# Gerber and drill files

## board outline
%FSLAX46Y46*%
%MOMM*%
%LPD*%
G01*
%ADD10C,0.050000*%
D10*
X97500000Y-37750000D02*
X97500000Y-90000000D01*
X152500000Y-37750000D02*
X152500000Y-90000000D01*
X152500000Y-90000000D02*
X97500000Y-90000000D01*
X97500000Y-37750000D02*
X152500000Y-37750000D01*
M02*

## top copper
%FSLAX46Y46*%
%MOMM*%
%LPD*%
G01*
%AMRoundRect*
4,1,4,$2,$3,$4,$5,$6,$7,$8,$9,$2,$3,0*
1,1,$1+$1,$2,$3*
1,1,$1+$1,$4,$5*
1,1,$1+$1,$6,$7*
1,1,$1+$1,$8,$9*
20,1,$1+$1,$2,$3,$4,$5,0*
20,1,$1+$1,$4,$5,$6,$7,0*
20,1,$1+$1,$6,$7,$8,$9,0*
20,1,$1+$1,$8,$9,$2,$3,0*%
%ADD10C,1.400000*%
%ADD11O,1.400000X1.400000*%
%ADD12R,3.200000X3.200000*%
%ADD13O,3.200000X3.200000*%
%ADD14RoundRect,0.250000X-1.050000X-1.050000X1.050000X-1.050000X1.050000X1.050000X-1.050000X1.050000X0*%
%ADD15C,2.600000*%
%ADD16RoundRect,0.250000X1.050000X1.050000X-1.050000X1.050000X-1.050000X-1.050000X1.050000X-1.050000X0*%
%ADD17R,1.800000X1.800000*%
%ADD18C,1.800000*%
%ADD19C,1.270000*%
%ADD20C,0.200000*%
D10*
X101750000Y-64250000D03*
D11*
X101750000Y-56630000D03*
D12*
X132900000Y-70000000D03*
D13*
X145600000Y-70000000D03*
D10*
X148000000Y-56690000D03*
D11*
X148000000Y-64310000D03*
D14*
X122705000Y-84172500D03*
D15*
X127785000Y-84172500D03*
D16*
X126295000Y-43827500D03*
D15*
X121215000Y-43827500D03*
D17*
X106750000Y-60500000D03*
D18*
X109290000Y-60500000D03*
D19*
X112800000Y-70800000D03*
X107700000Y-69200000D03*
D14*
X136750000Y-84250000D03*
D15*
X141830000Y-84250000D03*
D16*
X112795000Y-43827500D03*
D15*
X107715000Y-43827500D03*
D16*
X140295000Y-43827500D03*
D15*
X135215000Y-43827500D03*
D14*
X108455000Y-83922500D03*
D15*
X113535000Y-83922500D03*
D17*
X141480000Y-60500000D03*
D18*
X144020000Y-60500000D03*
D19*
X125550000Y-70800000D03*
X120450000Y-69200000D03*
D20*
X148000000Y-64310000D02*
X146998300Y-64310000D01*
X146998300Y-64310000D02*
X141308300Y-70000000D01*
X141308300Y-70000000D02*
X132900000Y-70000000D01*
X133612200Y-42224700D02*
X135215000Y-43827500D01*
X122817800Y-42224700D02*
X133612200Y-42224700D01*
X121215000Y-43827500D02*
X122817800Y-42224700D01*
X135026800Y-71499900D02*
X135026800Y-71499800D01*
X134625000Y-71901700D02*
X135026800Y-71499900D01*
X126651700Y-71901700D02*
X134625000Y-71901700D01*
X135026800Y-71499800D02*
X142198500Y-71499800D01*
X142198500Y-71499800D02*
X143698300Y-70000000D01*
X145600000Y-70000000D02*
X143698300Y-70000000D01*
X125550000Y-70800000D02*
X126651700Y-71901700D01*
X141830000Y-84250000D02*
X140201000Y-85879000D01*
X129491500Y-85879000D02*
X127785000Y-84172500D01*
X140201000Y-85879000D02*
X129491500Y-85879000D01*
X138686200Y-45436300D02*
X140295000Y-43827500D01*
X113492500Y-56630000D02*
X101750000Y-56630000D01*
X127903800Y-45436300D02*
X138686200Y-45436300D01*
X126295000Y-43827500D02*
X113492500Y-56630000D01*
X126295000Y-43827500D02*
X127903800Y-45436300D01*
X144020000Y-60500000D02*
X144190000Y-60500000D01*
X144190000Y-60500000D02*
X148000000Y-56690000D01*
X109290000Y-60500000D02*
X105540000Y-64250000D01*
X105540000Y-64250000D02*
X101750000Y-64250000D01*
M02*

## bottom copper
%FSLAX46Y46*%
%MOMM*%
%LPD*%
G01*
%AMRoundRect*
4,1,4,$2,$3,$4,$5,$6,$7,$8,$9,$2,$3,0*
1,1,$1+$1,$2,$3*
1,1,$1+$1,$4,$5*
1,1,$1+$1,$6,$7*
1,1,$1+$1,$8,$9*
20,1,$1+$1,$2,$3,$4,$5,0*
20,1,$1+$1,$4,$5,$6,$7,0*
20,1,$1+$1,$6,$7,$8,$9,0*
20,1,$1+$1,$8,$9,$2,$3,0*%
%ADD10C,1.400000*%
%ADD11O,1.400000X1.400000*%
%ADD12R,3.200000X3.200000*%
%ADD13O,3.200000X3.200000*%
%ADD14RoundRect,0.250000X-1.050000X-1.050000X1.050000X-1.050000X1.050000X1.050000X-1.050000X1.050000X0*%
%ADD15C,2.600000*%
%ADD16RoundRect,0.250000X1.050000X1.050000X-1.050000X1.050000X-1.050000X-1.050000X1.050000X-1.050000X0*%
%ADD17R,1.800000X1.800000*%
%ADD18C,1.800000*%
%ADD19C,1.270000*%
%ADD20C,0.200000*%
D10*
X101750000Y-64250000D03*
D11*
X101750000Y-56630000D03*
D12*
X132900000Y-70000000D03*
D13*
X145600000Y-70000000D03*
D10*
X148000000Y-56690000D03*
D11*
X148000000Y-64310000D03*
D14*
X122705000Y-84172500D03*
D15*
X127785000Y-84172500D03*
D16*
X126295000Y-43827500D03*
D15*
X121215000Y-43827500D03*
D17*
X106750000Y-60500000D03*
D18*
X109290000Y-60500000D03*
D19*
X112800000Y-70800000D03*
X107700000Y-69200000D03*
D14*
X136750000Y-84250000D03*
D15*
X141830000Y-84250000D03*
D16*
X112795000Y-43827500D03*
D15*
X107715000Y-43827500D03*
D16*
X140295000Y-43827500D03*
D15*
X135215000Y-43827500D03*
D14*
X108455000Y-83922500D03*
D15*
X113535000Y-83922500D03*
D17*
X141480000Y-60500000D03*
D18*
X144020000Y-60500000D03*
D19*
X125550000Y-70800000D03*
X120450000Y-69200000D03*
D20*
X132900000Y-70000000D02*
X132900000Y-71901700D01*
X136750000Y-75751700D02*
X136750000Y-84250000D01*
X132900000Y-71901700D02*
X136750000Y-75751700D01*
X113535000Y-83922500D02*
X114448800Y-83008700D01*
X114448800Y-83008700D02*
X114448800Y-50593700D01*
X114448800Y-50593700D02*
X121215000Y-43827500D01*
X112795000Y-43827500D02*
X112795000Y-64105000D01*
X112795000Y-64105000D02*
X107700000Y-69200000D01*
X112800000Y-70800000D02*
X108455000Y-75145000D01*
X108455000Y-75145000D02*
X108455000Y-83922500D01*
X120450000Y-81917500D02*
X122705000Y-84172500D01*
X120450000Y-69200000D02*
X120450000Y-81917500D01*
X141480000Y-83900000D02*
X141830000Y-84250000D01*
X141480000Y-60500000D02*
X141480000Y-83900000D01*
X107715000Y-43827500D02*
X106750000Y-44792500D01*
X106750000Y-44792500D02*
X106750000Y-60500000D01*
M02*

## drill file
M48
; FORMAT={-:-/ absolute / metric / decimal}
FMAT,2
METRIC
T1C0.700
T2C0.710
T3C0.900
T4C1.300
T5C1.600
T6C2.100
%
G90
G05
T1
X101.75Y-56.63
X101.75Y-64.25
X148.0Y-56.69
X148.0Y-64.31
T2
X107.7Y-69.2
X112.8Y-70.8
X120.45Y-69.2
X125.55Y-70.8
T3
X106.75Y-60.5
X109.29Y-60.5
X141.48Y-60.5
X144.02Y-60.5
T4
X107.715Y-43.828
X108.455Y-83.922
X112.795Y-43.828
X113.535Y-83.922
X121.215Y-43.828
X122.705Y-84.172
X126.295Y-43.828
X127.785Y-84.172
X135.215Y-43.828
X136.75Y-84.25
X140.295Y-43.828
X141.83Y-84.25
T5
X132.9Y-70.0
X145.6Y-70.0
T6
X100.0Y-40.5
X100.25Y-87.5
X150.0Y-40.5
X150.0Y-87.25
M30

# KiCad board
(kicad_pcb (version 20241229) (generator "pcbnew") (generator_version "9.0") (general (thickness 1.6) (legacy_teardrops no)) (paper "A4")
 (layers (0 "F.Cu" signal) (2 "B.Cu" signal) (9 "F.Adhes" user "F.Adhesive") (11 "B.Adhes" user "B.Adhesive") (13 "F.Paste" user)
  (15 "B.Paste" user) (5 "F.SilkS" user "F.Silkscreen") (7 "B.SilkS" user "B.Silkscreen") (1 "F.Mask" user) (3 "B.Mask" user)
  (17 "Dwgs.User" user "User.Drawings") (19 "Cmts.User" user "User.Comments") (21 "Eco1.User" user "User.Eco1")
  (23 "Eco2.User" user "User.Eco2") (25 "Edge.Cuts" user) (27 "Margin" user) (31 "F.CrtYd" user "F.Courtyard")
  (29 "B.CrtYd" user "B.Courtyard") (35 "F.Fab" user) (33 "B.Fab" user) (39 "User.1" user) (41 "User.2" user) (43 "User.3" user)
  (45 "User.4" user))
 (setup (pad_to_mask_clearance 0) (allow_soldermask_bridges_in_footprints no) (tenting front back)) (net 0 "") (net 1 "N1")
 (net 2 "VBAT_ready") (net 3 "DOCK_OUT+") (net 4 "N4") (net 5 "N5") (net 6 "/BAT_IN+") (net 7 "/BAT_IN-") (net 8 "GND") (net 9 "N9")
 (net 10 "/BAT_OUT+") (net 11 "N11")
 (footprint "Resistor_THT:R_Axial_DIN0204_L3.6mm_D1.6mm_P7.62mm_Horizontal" (layer "F.Cu") (at 101.75 64.25 90)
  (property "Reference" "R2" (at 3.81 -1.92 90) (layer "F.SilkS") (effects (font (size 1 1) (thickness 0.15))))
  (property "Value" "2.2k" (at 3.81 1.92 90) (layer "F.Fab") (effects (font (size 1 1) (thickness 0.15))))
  (pad "1" thru_hole circle (at 0 0 90) (size 1.4 1.4) (drill 0.7) (layers "*.Cu" "*.Mask") (remove_unused_layers no) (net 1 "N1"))
  (pad "2" thru_hole oval (at 7.62 0 90) (size 1.4 1.4) (drill 0.7) (layers "*.Cu" "*.Mask") (remove_unused_layers no) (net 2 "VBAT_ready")))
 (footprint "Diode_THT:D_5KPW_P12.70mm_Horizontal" (layer "F.Cu") (at 132.9 70)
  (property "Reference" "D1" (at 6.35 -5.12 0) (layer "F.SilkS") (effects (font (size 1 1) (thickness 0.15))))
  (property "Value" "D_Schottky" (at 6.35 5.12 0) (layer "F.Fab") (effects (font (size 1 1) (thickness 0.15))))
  (pad "1" thru_hole rect (at 0 0) (size 3.2 3.2) (drill 1.6) (layers "*.Cu" "*.Mask") (remove_unused_layers no) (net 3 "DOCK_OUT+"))
  (pad "2" thru_hole oval (at 12.7 0) (size 3.2 3.2) (drill 1.6) (layers "*.Cu" "*.Mask") (remove_unused_layers no) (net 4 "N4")))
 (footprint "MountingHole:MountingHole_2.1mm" (layer "F.Cu") (at 100.25 87.5)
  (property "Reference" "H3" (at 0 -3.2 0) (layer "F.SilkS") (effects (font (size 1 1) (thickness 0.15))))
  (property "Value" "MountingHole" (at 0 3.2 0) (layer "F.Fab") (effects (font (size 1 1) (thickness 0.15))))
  (pad "" np_thru_hole circle (at 0 0) (size 2.1 2.1) (drill 2.1) (layers "*.Cu" "*.Mask")))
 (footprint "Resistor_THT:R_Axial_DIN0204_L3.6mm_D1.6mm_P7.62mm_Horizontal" (layer "F.Cu") (at 148 56.69 -90)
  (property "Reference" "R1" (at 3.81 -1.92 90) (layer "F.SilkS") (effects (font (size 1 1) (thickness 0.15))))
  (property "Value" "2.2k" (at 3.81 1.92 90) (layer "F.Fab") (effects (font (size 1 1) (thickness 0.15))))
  (pad "1" thru_hole circle (at 0 0 270) (size 1.4 1.4) (drill 0.7) (layers "*.Cu" "*.Mask") (remove_unused_layers no) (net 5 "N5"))
  (pad "2" thru_hole oval (at 7.62 0 270) (size 1.4 1.4) (drill 0.7) (layers "*.Cu" "*.Mask") (remove_unused_layers no) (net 3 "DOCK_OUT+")))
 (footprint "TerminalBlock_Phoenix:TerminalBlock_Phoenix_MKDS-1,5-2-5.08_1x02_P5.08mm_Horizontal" (layer "F.Cu") (at 122.705 84.1725)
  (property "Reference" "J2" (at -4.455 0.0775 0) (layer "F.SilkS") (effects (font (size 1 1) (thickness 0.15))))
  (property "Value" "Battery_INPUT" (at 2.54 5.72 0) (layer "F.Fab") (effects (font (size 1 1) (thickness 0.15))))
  (pad "1" thru_hole roundrect (at 0 0) (size 2.6 2.6) (drill 1.3) (layers "*.Cu" "*.Mask") (remove_unused_layers no)
   (roundrect_rratio 0.096154) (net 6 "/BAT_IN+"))
  (pad "2" thru_hole circle (at 5.08 0) (size 2.6 2.6) (drill 1.3) (layers "*.Cu" "*.Mask") (remove_unused_layers no) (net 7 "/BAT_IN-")))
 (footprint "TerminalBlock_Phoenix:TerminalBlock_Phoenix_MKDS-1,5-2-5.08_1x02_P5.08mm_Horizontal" (layer "F.Cu") (at 126.295 43.8275 180)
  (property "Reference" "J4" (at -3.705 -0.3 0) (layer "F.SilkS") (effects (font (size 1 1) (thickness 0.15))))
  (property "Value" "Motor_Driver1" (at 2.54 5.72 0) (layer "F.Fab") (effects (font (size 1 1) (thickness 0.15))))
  (pad "1" thru_hole roundrect (at 0 0 180) (size 2.6 2.6) (drill 1.3) (layers "*.Cu" "*.Mask") (remove_unused_layers no)
   (roundrect_rratio 0.096154) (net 2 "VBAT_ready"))
  (pad "2" thru_hole circle (at 5.08 0 180) (size 2.6 2.6) (drill 1.3) (layers "*.Cu" "*.Mask") (remove_unused_layers no) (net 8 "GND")))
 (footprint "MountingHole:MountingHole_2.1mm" (layer "F.Cu") (at 150 40.5)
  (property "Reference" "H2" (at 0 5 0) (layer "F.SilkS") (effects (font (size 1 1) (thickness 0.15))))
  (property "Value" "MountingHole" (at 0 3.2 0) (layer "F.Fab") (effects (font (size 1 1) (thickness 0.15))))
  (pad "" np_thru_hole circle (at 0 0) (size 2.1 2.1) (drill 2.1) (layers "*.Cu" "*.Mask")))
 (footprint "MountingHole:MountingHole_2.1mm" (layer "F.Cu") (at 100 40.5)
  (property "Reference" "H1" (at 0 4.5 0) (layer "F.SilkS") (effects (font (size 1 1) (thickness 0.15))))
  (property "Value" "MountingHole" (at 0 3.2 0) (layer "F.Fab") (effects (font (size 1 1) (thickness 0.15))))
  (pad "" np_thru_hole circle (at 0 0) (size 2.1 2.1) (drill 2.1) (layers "*.Cu" "*.Mask")))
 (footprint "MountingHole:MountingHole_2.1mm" (layer "F.Cu") (at 150 87.25)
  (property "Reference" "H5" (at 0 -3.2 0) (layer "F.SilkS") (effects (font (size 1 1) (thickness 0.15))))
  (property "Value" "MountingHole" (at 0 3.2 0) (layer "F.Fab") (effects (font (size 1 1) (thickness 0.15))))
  (pad "" np_thru_hole circle (at 0 0) (size 2.1 2.1) (drill 2.1) (layers "*.Cu" "*.Mask")))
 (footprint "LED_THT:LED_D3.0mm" (layer "F.Cu") (at 106.75 60.5)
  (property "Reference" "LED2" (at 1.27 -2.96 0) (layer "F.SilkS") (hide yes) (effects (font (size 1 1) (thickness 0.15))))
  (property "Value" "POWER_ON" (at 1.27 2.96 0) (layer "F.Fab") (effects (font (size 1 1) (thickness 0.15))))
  (pad "1" thru_hole rect (at 0 0) (size 1.8 1.8) (drill 0.9) (layers "*.Cu" "*.Mask") (remove_unused_layers no) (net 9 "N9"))
  (pad "2" thru_hole circle (at 2.54 0) (size 1.8 1.8) (drill 0.9) (layers "*.Cu" "*.Mask") (remove_unused_layers no) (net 1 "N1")))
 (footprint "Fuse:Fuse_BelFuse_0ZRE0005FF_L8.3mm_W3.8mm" (layer "F.Cu") (at 112.8 70.8 180)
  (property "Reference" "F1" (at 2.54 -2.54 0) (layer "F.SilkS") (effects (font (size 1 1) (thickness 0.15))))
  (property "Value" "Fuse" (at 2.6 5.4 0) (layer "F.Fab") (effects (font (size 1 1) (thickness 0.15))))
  (pad "1" thru_hole circle (at 0 0 180) (size 1.27 1.27) (drill 0.71) (layers "*.Cu" "*.Mask") (remove_unused_layers no)
   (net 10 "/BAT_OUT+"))
  (pad "2" thru_hole circle (at 5.1 1.6 180) (size 1.27 1.27) (drill 0.71) (layers "*.Cu" "*.Mask") (remove_unused_layers no) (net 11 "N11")))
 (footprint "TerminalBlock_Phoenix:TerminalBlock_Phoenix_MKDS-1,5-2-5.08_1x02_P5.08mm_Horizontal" (layer "F.Cu") (at 136.75 84.25)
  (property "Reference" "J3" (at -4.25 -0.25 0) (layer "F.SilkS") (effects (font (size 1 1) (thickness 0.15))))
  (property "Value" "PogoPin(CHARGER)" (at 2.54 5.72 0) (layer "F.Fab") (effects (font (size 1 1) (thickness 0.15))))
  (pad "1" thru_hole roundrect (at 0 0) (size 2.6 2.6) (drill 1.3) (layers "*.Cu" "*.Mask") (remove_unused_layers no)
   (roundrect_rratio 0.096154) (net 3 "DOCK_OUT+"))
  (pad "2" thru_hole circle (at 5.08 0) (size 2.6 2.6) (drill 1.3) (layers "*.Cu" "*.Mask") (remove_unused_layers no) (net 7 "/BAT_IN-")))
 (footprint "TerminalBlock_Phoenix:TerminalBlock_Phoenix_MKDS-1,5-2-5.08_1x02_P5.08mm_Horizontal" (layer "F.Cu") (at 112.795 43.8275 180)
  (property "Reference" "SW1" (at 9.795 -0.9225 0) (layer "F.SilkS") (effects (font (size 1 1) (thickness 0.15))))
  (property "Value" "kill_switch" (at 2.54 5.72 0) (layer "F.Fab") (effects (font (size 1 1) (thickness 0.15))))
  (pad "1" thru_hole roundrect (at 0 0 180) (size 2.6 2.6) (drill 1.3) (layers "*.Cu" "*.Mask") (remove_unused_layers no)
   (roundrect_rratio 0.096154) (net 11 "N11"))
  (pad "2" thru_hole circle (at 5.08 0 180) (size 2.6 2.6) (drill 1.3) (layers "*.Cu" "*.Mask") (remove_unused_layers no) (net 9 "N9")))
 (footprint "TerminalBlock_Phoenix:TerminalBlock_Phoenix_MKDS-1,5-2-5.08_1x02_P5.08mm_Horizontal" (layer "F.Cu") (at 140.295 43.8275 180)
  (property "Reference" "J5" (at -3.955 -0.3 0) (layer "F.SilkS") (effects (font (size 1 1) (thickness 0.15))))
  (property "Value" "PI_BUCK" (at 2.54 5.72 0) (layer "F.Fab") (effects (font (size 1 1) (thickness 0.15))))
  (pad "1" thru_hole roundrect (at 0 0 180) (size 2.6 2.6) (drill 1.3) (layers "*.Cu" "*.Mask") (remove_unused_layers no)
   (roundrect_rratio 0.096154) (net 2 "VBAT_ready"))
  (pad "2" thru_hole circle (at 5.08 0 180) (size 2.6 2.6) (drill 1.3) (layers "*.Cu" "*.Mask") (remove_unused_layers no) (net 8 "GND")))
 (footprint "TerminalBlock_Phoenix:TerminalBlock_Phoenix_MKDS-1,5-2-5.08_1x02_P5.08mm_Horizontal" (layer "F.Cu") (at 108.455 83.9225)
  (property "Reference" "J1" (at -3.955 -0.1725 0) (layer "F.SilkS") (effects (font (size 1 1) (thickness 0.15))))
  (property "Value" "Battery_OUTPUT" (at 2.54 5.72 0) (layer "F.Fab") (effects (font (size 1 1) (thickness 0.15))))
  (pad "1" thru_hole roundrect (at 0 0) (size 2.6 2.6) (drill 1.3) (layers "*.Cu" "*.Mask") (remove_unused_layers no)
   (roundrect_rratio 0.096154) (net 10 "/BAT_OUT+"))
  (pad "2" thru_hole circle (at 5.08 0) (size 2.6 2.6) (drill 1.3) (layers "*.Cu" "*.Mask") (remove_unused_layers no) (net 8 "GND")))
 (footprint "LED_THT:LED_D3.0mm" (layer "F.Cu") (at 141.48 60.5)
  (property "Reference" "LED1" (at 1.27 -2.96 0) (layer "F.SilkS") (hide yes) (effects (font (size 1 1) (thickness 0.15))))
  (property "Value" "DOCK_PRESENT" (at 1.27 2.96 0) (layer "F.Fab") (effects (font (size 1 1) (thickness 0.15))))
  (pad "1" thru_hole rect (at 0 0) (size 1.8 1.8) (drill 0.9) (layers "*.Cu" "*.Mask") (remove_unused_layers no) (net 7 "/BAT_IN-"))
  (pad "2" thru_hole circle (at 2.54 0) (size 1.8 1.8) (drill 0.9) (layers "*.Cu" "*.Mask") (remove_unused_layers no) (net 5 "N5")))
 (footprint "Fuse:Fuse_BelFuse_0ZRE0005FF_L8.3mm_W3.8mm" (layer "F.Cu") (at 125.55 70.8 180)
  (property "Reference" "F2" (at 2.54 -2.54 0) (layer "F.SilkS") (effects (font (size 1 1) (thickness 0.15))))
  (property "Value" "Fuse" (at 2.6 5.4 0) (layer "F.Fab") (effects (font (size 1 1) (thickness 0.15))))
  (pad "1" thru_hole circle (at 0 0 180) (size 1.27 1.27) (drill 0.71) (layers "*.Cu" "*.Mask") (remove_unused_layers no) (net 4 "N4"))
  (pad "2" thru_hole circle (at 5.1 1.6 180) (size 1.27 1.27) (drill 0.71) (layers "*.Cu" "*.Mask") (remove_unused_layers no)
   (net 6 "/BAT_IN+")))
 (gr_line (start 97.5 37.75) (end 97.5 90) (stroke (width 0.05) (type default)) (layer "Edge.Cuts"))
 (gr_line (start 152.5 37.75) (end 152.5 90) (stroke (width 0.05) (type default)) (layer "Edge.Cuts"))
 (gr_line (start 152.5 90) (end 97.5 90) (stroke (width 0.05) (type default)) (layer "Edge.Cuts"))
 (gr_line (start 97.5 37.75) (end 152.5 37.75) (stroke (width 0.05) (type default)) (layer "Edge.Cuts"))
 (segment (start 148 64.31) (end 146.9983 64.31) (width 0.2) (layer "F.Cu") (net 3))
 (segment (start 146.9983 64.31) (end 141.3083 70) (width 0.2) (layer "F.Cu") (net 3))
 (segment (start 141.3083 70) (end 132.9 70) (width 0.2) (layer "F.Cu") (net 3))
 (segment (start 132.9 70) (end 132.9 71.9017) (width 0.2) (layer "B.Cu") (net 3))
 (segment (start 136.75 75.7517) (end 136.75 84.25) (width 0.2) (layer "B.Cu") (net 3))
 (segment (start 132.9 71.9017) (end 136.75 75.7517) (width 0.2) (layer "B.Cu") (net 3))
 (segment (start 133.6122 42.2247) (end 135.215 43.8275) (width 0.2) (layer "F.Cu") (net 8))
 (segment (start 122.8178 42.2247) (end 133.6122 42.2247) (width 0.2) (layer "F.Cu") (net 8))
 (segment (start 121.215 43.8275) (end 122.8178 42.2247) (width 0.2) (layer "F.Cu") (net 8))
 (segment (start 113.535 83.9225) (end 114.4488 83.0087) (width 0.2) (layer "B.Cu") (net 8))
 (segment (start 114.4488 83.0087) (end 114.4488 50.5937) (width 0.2) (layer "B.Cu") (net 8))
 (segment (start 114.4488 50.5937) (end 121.215 43.8275) (width 0.2) (layer "B.Cu") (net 8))
 (segment (start 135.0268 71.4999) (end 135.0268 71.4998) (width 0.2) (layer "F.Cu") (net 4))
 (segment (start 134.625 71.9017) (end 135.0268 71.4999) (width 0.2) (layer "F.Cu") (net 4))
 (segment (start 126.6517 71.9017) (end 134.625 71.9017) (width 0.2) (layer "F.Cu") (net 4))
 (segment (start 135.0268 71.4998) (end 142.1985 71.4998) (width 0.2) (layer "F.Cu") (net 4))
 (segment (start 142.1985 71.4998) (end 143.6983 70) (width 0.2) (layer "F.Cu") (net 4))
 (segment (start 145.6 70) (end 143.6983 70) (width 0.2) (layer "F.Cu") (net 4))
 (segment (start 125.55 70.8) (end 126.6517 71.9017) (width 0.2) (layer "F.Cu") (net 4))
 (segment (start 112.795 43.8275) (end 112.795 64.105) (width 0.2) (layer "B.Cu") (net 11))
 (segment (start 112.795 64.105) (end 107.7 69.2) (width 0.2) (layer "B.Cu") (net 11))
 (segment (start 112.8 70.8) (end 108.455 75.145) (width 0.2) (layer "B.Cu") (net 10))
 (segment (start 108.455 75.145) (end 108.455 83.9225) (width 0.2) (layer "B.Cu") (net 10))
 (segment (start 120.45 81.9175) (end 122.705 84.1725) (width 0.2) (layer "B.Cu") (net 6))
 (segment (start 120.45 69.2) (end 120.45 81.9175) (width 0.2) (layer "B.Cu") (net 6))
 (segment (start 141.83 84.25) (end 140.201 85.879) (width 0.2) (layer "F.Cu") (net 7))
 (segment (start 129.4915 85.879) (end 127.785 84.1725) (width 0.2) (layer "F.Cu") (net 7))
 (segment (start 140.201 85.879) (end 129.4915 85.879) (width 0.2) (layer "F.Cu") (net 7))
 (segment (start 141.48 83.9) (end 141.83 84.25) (width 0.2) (layer "B.Cu") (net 7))
 (segment (start 141.48 60.5) (end 141.48 83.9) (width 0.2) (layer "B.Cu") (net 7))
 (segment (start 138.6862 45.4363) (end 140.295 43.8275) (width 0.2) (layer "F.Cu") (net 2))
 (segment (start 113.4925 56.63) (end 101.75 56.63) (width 0.2) (layer "F.Cu") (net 2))
 (segment (start 127.9038 45.4363) (end 138.6862 45.4363) (width 0.2) (layer "F.Cu") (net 2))
 (segment (start 126.295 43.8275) (end 113.4925 56.63) (width 0.2) (layer "F.Cu") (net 2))
 (segment (start 126.295 43.8275) (end 127.9038 45.4363) (width 0.2) (layer "F.Cu") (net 2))
 (segment (start 144.02 60.5) (end 144.19 60.5) (width 0.2) (layer "F.Cu") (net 5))
 (segment (start 144.19 60.5) (end 148 56.69) (width 0.2) (layer "F.Cu") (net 5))
 (segment (start 107.715 43.8275) (end 106.75 44.7925) (width 0.2) (layer "B.Cu") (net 9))
 (segment (start 106.75 44.7925) (end 106.75 60.5) (width 0.2) (layer "B.Cu") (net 9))
 (segment (start 109.29 60.5) (end 105.54 64.25) (width 0.2) (layer "F.Cu") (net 1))
 (segment (start 105.54 64.25) (end 101.75 64.25) (width 0.2) (layer "F.Cu") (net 1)))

